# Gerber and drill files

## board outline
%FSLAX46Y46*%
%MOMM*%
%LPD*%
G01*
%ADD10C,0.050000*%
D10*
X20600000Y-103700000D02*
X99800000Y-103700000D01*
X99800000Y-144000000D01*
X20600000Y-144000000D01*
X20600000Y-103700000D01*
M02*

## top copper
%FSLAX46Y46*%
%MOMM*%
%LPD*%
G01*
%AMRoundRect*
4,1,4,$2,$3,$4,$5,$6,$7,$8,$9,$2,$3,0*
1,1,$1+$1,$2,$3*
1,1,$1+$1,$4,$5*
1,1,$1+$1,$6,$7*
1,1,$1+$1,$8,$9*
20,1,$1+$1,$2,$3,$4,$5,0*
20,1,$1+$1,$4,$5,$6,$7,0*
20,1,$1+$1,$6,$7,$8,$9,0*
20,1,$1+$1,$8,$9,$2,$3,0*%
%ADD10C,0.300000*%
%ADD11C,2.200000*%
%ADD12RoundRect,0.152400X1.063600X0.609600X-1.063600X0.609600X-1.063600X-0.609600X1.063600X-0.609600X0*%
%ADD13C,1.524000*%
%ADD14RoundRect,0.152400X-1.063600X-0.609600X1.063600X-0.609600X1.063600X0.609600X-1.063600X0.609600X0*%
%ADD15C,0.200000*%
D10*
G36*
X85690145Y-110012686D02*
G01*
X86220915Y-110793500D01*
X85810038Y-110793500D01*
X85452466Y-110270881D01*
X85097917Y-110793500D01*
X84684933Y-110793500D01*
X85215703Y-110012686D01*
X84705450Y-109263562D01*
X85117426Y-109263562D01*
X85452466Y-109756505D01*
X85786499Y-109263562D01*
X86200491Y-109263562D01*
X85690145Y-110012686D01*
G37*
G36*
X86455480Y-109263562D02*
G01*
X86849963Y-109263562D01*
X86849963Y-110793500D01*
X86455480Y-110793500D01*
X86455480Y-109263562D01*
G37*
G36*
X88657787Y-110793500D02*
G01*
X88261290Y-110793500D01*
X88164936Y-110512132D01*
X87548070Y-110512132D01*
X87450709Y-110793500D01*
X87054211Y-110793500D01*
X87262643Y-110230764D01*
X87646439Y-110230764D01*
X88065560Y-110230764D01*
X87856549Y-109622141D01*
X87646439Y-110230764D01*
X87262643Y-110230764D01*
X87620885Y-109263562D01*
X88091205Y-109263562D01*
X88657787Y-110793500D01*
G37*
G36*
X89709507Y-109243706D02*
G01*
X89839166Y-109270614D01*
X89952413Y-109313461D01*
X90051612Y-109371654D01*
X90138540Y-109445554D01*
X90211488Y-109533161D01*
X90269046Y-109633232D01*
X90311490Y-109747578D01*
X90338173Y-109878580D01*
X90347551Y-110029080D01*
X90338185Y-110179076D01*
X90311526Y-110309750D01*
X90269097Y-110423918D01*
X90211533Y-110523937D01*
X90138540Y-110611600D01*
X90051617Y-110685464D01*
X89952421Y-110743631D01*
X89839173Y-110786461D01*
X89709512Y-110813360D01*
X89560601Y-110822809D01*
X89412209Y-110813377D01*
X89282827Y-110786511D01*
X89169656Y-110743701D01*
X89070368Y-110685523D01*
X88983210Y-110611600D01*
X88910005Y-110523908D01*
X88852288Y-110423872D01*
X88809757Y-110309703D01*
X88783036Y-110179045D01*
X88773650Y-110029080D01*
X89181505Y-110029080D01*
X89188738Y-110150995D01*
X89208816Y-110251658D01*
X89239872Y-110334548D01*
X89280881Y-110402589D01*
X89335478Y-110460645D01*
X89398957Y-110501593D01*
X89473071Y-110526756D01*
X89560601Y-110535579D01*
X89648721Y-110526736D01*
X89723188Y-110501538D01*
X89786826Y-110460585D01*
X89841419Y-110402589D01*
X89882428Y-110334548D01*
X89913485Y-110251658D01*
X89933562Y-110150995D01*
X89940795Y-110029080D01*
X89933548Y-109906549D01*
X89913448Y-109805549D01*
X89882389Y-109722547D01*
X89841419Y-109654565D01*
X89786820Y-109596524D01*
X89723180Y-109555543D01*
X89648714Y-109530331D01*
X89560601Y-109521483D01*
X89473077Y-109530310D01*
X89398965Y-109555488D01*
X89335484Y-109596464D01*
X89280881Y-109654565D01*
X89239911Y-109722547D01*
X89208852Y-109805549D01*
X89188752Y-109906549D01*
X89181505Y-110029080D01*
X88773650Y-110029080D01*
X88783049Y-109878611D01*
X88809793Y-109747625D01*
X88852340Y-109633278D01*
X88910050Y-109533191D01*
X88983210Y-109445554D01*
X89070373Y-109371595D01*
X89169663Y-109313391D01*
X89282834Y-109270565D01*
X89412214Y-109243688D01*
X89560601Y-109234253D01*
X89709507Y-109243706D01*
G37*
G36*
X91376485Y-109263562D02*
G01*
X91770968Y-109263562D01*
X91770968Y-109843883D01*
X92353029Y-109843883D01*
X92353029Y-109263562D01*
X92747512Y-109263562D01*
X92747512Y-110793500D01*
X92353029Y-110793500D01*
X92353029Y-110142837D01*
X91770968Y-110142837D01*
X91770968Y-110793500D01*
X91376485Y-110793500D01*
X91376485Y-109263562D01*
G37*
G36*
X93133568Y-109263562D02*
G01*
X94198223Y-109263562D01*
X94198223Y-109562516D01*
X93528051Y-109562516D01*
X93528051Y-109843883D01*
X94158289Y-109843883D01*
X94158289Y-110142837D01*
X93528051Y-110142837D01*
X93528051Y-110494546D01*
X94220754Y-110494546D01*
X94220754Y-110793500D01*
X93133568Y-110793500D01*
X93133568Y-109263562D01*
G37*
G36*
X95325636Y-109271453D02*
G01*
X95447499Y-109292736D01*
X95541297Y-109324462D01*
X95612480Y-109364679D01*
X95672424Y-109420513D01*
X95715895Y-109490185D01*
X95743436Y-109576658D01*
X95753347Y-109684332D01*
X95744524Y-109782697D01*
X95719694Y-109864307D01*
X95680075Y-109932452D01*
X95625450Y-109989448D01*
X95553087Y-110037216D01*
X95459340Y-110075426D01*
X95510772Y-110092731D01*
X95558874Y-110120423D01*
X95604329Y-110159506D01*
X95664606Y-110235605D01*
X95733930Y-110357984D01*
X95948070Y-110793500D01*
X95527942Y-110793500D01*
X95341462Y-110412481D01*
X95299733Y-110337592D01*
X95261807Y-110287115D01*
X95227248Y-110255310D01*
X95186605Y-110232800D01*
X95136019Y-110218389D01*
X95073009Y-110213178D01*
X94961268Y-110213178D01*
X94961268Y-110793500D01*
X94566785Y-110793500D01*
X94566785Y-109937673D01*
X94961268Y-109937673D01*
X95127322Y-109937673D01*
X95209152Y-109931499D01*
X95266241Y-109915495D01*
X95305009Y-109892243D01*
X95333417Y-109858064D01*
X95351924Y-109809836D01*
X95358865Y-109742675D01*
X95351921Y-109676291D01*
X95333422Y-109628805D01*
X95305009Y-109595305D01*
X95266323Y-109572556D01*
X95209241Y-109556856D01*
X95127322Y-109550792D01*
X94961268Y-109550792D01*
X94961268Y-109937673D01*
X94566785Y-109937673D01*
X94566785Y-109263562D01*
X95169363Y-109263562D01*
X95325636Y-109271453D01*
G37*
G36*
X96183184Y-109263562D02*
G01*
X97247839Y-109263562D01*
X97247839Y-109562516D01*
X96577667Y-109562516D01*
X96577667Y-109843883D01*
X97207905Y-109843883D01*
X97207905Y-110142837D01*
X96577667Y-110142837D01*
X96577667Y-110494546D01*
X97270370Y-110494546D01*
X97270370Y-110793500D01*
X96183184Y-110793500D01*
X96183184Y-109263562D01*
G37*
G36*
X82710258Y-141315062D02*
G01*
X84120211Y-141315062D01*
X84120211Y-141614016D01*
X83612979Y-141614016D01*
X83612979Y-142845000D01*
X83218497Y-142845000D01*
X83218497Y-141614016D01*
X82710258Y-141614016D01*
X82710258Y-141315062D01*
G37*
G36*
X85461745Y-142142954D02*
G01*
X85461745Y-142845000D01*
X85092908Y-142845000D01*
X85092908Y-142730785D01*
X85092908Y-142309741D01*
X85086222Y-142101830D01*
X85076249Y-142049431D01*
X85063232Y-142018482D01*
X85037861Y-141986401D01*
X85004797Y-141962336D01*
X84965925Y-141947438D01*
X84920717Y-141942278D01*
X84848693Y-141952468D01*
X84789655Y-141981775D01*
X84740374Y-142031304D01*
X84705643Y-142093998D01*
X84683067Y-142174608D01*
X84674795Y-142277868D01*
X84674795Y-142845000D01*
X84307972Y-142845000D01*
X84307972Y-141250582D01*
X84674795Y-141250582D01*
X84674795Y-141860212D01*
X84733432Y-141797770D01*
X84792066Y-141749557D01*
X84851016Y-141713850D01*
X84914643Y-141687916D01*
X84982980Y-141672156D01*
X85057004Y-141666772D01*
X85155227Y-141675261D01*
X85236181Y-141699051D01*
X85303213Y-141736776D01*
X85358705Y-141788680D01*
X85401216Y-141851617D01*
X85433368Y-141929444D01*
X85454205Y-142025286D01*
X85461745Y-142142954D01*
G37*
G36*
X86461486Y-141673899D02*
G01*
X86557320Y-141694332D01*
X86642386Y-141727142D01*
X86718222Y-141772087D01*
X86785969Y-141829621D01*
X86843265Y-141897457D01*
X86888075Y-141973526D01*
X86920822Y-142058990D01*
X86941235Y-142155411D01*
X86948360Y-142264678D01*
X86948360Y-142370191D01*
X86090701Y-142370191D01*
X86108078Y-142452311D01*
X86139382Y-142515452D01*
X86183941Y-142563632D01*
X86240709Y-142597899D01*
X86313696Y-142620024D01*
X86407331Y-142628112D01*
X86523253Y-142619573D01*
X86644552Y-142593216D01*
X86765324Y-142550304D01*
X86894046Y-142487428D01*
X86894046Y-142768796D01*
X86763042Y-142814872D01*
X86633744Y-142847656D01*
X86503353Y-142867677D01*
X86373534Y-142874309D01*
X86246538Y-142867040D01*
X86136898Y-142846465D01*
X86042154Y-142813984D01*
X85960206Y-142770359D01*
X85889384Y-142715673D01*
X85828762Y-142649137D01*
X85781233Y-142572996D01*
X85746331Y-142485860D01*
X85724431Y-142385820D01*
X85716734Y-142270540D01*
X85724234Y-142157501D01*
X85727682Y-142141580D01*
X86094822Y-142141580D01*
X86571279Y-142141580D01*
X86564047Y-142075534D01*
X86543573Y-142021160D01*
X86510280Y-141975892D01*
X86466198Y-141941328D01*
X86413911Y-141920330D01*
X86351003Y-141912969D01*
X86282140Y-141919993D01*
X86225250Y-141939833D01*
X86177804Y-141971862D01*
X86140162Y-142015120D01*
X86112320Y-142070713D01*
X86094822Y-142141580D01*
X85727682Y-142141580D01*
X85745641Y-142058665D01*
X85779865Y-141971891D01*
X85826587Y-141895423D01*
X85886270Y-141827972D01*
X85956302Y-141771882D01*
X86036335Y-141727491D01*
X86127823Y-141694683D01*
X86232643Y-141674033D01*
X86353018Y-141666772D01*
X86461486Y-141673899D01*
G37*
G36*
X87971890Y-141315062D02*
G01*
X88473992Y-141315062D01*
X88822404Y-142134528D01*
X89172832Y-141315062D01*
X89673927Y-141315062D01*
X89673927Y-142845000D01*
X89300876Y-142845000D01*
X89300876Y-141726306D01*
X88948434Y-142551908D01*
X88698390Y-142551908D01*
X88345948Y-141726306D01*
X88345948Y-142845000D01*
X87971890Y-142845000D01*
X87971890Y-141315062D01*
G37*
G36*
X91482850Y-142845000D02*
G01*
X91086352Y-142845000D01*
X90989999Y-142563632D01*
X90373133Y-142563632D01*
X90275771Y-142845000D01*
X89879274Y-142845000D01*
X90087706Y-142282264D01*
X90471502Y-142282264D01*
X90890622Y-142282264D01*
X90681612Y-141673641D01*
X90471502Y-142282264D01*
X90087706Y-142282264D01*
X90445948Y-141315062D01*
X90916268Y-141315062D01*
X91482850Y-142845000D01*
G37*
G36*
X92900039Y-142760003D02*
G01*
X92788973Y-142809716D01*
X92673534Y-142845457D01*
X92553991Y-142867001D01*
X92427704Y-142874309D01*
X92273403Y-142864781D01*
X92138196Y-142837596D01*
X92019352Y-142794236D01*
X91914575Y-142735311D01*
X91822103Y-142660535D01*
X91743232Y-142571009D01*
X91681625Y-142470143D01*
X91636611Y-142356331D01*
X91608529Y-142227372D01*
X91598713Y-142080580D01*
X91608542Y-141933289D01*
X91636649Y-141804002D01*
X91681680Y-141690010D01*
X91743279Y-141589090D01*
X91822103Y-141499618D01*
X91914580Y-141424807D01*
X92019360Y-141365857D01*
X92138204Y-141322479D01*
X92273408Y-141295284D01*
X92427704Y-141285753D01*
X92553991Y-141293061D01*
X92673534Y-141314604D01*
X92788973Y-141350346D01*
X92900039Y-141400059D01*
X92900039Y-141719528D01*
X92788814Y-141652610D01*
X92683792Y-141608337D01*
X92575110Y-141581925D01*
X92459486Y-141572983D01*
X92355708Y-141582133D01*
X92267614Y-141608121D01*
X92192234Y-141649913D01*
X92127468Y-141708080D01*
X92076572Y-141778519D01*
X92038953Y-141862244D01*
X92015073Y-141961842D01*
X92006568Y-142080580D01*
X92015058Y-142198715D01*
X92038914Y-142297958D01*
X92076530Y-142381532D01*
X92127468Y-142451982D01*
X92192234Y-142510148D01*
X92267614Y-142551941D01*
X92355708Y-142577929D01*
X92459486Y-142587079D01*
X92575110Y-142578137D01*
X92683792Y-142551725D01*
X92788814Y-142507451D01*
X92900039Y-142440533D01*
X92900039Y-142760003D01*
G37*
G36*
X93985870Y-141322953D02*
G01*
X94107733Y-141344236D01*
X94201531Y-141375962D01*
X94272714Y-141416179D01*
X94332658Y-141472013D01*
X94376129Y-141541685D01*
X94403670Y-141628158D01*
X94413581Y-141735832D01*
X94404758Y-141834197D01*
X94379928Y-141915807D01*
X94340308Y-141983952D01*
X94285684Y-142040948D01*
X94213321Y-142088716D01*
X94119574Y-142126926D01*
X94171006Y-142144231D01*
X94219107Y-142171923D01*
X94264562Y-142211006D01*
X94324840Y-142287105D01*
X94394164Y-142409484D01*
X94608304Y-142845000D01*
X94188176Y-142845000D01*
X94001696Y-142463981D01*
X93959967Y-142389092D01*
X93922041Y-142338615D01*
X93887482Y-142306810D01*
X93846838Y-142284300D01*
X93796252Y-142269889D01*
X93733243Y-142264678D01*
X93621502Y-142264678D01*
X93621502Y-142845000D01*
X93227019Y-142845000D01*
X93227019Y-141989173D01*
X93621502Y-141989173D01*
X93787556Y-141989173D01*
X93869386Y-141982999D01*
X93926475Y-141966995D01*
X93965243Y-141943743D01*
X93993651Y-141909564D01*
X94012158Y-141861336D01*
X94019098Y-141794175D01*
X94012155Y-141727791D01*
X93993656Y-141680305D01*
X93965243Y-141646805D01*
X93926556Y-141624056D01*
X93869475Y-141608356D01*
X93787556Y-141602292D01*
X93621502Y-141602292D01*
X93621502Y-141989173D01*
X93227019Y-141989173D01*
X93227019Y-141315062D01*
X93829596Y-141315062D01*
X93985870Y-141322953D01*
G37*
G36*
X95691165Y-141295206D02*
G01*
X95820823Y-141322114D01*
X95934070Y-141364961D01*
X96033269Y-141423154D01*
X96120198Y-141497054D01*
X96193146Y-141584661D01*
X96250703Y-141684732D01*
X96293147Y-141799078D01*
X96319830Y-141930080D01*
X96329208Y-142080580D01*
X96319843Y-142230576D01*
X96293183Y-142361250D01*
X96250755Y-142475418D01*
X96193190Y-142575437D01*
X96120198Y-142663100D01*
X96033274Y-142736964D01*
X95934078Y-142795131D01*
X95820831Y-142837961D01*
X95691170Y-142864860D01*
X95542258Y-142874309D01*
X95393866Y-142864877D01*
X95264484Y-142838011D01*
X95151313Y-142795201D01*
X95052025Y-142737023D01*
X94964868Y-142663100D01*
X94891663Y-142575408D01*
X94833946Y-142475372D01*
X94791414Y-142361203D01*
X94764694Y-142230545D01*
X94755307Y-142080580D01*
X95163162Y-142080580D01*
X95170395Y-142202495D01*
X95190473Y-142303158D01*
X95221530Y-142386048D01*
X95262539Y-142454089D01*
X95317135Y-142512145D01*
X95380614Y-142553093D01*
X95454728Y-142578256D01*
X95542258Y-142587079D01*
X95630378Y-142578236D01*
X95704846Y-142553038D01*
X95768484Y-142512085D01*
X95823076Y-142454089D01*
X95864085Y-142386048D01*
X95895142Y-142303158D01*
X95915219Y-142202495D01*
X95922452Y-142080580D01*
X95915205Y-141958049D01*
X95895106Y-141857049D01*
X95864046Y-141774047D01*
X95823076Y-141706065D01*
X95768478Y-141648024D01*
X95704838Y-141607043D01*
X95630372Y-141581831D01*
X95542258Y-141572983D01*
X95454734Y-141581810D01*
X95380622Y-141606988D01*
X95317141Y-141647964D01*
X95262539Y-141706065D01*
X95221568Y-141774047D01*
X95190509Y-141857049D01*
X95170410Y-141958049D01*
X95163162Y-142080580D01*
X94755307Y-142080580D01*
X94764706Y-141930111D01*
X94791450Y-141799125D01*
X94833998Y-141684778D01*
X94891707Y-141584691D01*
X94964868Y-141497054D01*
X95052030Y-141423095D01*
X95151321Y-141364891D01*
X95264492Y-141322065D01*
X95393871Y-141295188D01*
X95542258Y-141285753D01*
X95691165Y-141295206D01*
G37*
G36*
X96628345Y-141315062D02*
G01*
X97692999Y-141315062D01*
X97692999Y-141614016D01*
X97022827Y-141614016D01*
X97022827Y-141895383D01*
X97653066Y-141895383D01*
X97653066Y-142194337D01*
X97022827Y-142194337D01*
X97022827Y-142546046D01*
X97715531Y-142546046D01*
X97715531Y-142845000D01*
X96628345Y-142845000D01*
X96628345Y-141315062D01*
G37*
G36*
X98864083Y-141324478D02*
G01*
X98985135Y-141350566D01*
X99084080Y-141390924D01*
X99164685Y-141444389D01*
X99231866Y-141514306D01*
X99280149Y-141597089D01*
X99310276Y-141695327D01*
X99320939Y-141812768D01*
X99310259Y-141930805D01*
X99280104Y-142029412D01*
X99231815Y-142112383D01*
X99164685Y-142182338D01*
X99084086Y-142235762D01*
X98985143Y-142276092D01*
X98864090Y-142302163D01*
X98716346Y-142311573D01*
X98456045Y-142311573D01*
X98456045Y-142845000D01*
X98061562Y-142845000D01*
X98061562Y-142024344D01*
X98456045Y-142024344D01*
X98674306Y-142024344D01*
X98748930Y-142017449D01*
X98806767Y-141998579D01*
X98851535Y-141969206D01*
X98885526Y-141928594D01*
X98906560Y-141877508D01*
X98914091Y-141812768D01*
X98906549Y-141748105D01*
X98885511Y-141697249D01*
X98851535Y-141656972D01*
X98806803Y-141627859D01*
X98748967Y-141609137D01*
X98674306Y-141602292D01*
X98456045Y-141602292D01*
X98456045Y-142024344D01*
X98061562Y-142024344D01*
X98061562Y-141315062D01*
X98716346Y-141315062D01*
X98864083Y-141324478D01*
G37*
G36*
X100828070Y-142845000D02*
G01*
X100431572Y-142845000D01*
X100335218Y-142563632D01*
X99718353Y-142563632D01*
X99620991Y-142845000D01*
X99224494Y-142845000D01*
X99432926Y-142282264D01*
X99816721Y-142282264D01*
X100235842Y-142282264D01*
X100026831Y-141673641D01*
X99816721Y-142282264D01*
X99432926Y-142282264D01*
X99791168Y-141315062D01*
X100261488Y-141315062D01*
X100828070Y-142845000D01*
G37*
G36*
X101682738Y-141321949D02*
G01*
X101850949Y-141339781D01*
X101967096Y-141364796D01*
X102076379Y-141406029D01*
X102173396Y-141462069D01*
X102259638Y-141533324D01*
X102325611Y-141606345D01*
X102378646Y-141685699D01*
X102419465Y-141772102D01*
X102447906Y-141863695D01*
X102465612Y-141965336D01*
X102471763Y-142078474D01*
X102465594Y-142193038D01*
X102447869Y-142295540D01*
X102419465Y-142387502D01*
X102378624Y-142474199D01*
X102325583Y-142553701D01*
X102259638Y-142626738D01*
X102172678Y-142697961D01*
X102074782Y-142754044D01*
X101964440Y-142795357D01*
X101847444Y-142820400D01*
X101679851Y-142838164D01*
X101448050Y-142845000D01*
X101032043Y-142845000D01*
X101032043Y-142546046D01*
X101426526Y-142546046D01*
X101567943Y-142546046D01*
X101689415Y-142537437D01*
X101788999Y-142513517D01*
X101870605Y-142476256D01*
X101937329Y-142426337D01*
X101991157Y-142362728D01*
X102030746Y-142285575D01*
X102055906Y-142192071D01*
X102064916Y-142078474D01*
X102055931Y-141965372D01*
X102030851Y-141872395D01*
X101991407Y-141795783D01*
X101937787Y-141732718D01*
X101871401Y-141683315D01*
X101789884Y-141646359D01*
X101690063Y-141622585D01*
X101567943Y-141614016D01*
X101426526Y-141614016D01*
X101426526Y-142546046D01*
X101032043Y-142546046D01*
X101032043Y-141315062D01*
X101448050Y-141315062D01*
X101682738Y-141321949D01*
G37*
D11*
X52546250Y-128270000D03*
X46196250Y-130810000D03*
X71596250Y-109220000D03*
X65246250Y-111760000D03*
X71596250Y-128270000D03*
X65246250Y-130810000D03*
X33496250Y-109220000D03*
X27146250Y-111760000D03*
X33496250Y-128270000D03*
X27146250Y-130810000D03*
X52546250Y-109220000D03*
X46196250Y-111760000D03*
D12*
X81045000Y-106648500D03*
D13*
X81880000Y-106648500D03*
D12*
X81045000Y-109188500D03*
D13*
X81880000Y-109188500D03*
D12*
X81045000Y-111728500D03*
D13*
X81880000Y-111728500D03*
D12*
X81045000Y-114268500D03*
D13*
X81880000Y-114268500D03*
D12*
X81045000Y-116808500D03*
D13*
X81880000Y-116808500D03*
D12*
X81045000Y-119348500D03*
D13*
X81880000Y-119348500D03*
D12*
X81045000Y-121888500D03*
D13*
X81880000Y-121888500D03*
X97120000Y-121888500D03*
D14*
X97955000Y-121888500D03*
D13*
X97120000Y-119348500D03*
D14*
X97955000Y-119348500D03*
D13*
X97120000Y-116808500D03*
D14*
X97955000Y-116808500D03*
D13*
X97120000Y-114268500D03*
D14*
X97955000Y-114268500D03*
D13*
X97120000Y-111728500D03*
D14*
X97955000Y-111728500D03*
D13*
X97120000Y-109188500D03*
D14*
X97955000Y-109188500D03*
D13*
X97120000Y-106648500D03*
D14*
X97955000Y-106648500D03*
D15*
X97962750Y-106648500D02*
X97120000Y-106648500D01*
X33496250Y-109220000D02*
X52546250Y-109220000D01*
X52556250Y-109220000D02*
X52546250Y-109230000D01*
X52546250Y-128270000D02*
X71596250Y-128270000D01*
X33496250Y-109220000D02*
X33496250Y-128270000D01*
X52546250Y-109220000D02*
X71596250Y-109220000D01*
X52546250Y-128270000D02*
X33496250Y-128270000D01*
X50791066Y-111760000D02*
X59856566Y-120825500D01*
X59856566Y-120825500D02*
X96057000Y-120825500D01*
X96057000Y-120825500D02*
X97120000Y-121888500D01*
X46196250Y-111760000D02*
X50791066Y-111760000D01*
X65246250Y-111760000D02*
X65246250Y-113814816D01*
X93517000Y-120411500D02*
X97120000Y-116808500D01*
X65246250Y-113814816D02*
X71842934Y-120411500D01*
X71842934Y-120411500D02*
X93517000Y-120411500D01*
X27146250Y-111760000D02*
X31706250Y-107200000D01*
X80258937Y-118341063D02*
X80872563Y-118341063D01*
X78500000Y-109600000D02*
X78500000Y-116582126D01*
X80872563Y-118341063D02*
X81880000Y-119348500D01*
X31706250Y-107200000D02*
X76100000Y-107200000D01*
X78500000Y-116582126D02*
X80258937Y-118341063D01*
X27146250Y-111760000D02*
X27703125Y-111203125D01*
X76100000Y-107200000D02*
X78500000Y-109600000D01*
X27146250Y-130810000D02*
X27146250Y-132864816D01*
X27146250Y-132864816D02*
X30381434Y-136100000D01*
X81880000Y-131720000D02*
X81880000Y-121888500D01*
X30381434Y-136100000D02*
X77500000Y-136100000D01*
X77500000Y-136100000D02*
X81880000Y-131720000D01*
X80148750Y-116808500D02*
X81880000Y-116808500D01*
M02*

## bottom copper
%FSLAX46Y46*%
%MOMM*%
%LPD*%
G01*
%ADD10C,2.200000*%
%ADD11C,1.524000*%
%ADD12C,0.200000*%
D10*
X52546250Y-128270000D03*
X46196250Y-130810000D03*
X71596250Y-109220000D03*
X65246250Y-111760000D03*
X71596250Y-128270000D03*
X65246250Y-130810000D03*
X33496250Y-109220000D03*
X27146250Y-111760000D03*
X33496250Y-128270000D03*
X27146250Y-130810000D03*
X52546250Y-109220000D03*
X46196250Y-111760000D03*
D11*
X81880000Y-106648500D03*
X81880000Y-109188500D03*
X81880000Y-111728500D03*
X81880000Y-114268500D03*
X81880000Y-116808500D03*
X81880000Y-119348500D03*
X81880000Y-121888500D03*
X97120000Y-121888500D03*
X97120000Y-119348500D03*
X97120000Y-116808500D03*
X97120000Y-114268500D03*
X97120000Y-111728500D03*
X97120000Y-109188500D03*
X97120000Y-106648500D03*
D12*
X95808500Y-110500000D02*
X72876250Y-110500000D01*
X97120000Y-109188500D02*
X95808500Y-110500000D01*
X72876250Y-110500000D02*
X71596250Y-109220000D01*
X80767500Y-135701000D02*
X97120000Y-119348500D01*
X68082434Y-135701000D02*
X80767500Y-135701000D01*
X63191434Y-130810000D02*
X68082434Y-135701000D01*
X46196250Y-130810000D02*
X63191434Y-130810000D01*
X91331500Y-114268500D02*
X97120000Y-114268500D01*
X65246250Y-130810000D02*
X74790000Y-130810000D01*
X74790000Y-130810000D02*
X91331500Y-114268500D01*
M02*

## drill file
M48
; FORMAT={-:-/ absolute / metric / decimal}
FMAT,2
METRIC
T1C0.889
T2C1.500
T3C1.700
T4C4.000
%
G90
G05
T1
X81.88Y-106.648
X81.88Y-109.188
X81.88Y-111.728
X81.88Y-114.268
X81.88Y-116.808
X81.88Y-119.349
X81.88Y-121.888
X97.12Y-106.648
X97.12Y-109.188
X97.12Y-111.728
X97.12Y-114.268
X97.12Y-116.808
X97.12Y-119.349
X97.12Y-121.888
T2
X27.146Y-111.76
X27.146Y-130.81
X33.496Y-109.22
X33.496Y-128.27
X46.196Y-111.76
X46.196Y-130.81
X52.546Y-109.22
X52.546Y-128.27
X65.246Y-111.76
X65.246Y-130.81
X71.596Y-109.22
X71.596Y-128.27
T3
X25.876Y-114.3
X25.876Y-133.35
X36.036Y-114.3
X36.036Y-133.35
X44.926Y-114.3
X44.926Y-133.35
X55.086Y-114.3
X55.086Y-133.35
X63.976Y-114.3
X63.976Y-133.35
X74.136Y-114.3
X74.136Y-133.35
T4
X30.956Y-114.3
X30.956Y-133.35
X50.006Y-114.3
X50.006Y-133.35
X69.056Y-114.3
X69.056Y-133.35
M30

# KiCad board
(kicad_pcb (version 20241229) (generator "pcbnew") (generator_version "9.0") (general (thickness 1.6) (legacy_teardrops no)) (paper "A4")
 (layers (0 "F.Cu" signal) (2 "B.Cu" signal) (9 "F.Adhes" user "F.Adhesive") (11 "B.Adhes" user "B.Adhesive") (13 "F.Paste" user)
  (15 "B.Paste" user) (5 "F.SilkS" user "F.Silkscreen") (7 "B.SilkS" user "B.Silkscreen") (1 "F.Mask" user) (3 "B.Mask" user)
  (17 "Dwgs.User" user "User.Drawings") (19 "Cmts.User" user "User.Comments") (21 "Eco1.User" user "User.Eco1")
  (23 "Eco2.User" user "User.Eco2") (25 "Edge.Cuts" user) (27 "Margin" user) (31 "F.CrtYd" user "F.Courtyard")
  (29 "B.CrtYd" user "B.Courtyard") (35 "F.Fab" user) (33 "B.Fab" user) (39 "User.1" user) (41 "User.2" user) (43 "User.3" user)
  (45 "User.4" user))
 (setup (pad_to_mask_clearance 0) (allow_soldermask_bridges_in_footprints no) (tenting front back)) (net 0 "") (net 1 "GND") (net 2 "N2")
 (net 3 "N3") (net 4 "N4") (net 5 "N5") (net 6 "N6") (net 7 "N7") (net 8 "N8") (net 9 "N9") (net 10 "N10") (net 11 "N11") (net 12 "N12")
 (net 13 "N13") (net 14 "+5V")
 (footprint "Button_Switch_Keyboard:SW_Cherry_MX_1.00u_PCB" (layer "F.Cu") (at 52.54625 128.27)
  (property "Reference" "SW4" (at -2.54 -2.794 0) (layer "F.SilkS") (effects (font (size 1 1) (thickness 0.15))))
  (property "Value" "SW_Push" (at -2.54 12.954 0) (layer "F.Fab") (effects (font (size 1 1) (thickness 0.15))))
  (pad "" np_thru_hole circle (at -7.62 5.08) (size 1.7 1.7) (drill 1.7) (layers "*.Cu" "*.Mask"))
  (pad "" np_thru_hole circle (at -2.54 5.08) (size 4 4) (drill 4) (layers "*.Cu" "*.Mask"))
  (pad "" np_thru_hole circle (at 2.54 5.08) (size 1.7 1.7) (drill 1.7) (layers "*.Cu" "*.Mask"))
  (pad "1" thru_hole circle (at 0 0) (size 2.2 2.2) (drill 1.5) (layers "*.Cu" "*.Mask") (remove_unused_layers no) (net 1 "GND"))
  (pad "2" thru_hole circle (at -6.35 2.54) (size 2.2 2.2) (drill 1.5) (layers "*.Cu" "*.Mask") (remove_unused_layers no) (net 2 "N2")))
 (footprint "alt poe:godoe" (layer "F.Cu") (at 90.7 131.5)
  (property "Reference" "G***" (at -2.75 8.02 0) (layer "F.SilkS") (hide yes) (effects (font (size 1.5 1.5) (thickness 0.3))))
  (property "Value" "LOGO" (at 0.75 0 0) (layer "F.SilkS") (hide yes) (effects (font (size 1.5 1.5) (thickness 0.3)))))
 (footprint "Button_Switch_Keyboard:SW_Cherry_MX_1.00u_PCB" (layer "F.Cu") (at 71.59625 109.22)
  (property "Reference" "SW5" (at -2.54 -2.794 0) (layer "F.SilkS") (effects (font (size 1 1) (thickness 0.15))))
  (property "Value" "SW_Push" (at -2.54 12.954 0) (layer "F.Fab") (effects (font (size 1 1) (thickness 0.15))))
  (pad "" np_thru_hole circle (at -7.62 5.08) (size 1.7 1.7) (drill 1.7) (layers "*.Cu" "*.Mask"))
  (pad "" np_thru_hole circle (at -2.54 5.08) (size 4 4) (drill 4) (layers "*.Cu" "*.Mask"))
  (pad "" np_thru_hole circle (at 2.54 5.08) (size 1.7 1.7) (drill 1.7) (layers "*.Cu" "*.Mask"))
  (pad "1" thru_hole circle (at 0 0) (size 2.2 2.2) (drill 1.5) (layers "*.Cu" "*.Mask") (remove_unused_layers no) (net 1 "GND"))
  (pad "2" thru_hole circle (at -6.35 2.54) (size 2.2 2.2) (drill 1.5) (layers "*.Cu" "*.Mask") (remove_unused_layers no) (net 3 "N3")))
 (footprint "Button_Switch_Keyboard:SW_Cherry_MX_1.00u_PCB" (layer "F.Cu") (at 71.59625 128.27)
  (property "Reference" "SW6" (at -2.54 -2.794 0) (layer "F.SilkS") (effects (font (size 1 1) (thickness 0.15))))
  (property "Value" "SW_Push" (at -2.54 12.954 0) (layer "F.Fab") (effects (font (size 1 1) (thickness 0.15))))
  (pad "" np_thru_hole circle (at -7.62 5.08) (size 1.7 1.7) (drill 1.7) (layers "*.Cu" "*.Mask"))
  (pad "" np_thru_hole circle (at -2.54 5.08) (size 4 4) (drill 4) (layers "*.Cu" "*.Mask"))
  (pad "" np_thru_hole circle (at 2.54 5.08) (size 1.7 1.7) (drill 1.7) (layers "*.Cu" "*.Mask"))
  (pad "1" thru_hole circle (at 0 0) (size 2.2 2.2) (drill 1.5) (layers "*.Cu" "*.Mask") (remove_unused_layers no) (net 1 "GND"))
  (pad "2" thru_hole circle (at -6.35 2.54) (size 2.2 2.2) (drill 1.5) (layers "*.Cu" "*.Mask") (remove_unused_layers no) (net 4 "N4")))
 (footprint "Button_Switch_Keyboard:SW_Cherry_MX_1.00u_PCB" (layer "F.Cu") (at 33.49625 109.22)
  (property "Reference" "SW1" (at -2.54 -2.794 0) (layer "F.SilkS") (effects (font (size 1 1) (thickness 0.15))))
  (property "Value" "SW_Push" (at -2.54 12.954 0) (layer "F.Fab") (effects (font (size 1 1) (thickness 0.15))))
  (pad "" np_thru_hole circle (at -7.62 5.08) (size 1.7 1.7) (drill 1.7) (layers "*.Cu" "*.Mask"))
  (pad "" np_thru_hole circle (at -2.54 5.08) (size 4 4) (drill 4) (layers "*.Cu" "*.Mask"))
  (pad "" np_thru_hole circle (at 2.54 5.08) (size 1.7 1.7) (drill 1.7) (layers "*.Cu" "*.Mask"))
  (pad "1" thru_hole circle (at 0 0) (size 2.2 2.2) (drill 1.5) (layers "*.Cu" "*.Mask") (remove_unused_layers no) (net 1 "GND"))
  (pad "2" thru_hole circle (at -6.35 2.54) (size 2.2 2.2) (drill 1.5) (layers "*.Cu" "*.Mask") (remove_unused_layers no) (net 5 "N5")))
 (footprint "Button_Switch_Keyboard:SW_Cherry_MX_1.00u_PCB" (layer "F.Cu") (at 33.49625 128.27)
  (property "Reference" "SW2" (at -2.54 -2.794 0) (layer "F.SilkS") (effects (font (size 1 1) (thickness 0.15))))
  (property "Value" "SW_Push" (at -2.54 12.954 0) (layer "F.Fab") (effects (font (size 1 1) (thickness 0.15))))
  (pad "" np_thru_hole circle (at -7.62 5.08) (size 1.7 1.7) (drill 1.7) (layers "*.Cu" "*.Mask"))
  (pad "" np_thru_hole circle (at -2.54 5.08) (size 4 4) (drill 4) (layers "*.Cu" "*.Mask"))
  (pad "" np_thru_hole circle (at 2.54 5.08) (size 1.7 1.7) (drill 1.7) (layers "*.Cu" "*.Mask"))
  (pad "1" thru_hole circle (at 0 0) (size 2.2 2.2) (drill 1.5) (layers "*.Cu" "*.Mask") (remove_unused_layers no) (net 1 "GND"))
  (pad "2" thru_hole circle (at -6.35 2.54) (size 2.2 2.2) (drill 1.5) (layers "*.Cu" "*.Mask") (remove_unused_layers no) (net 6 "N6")))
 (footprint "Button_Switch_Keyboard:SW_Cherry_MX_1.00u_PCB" (layer "F.Cu") (at 52.54625 109.22)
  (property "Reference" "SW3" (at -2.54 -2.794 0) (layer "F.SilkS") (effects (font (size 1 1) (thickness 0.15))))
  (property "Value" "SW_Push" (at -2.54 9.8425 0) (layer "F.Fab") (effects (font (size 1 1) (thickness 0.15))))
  (pad "" np_thru_hole circle (at -7.62 5.08) (size 1.7 1.7) (drill 1.7) (layers "*.Cu" "*.Mask"))
  (pad "" np_thru_hole circle (at -2.54 5.08) (size 4 4) (drill 4) (layers "*.Cu" "*.Mask"))
  (pad "" np_thru_hole circle (at 2.54 5.08) (size 1.7 1.7) (drill 1.7) (layers "*.Cu" "*.Mask"))
  (pad "1" thru_hole circle (at 0 0) (size 2.2 2.2) (drill 1.5) (layers "*.Cu" "*.Mask") (remove_unused_layers no) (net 1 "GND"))
  (pad "2" thru_hole circle (at -6.35 2.54) (size 2.2 2.2) (drill 1.5) (layers "*.Cu" "*.Mask") (remove_unused_layers no) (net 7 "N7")))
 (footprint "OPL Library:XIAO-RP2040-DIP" (layer "F.Cu") (at 89.5 114.2685)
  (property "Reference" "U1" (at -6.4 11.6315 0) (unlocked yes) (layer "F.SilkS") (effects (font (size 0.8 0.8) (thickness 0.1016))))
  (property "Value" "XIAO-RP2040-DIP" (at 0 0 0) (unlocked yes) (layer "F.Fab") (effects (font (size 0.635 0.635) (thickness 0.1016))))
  (pad "1" smd roundrect (at -8.455 -7.62 180) (size 2.432 1.524) (layers "F.Cu" "F.Mask") (roundrect_rratio 0.1) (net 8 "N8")
   (thermal_bridge_angle 45))
  (pad "1" thru_hole circle (at -7.62 -7.62 180) (size 1.524 1.524) (drill 0.889) (layers "*.Cu" "*.Mask") (remove_unused_layers no)
   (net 8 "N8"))
  (pad "2" smd roundrect (at -8.455 -5.08 180) (size 2.432 1.524) (layers "F.Cu" "F.Mask") (roundrect_rratio 0.1) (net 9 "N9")
   (thermal_bridge_angle 45))
  (pad "2" thru_hole circle (at -7.62 -5.08 180) (size 1.524 1.524) (drill 0.889) (layers "*.Cu" "*.Mask") (remove_unused_layers no)
   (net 9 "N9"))
  (pad "3" smd roundrect (at -8.455 -2.54 180) (size 2.432 1.524) (layers "F.Cu" "F.Mask") (roundrect_rratio 0.1) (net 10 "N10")
   (thermal_bridge_angle 45))
  (pad "3" thru_hole circle (at -7.62 -2.54 180) (size 1.524 1.524) (drill 0.889) (layers "*.Cu" "*.Mask") (remove_unused_layers no)
   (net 10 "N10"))
  (pad "4" smd roundrect (at -8.455 0 180) (size 2.432 1.524) (layers "F.Cu" "F.Mask") (roundrect_rratio 0.1) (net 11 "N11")
   (thermal_bridge_angle 45))
  (pad "4" thru_hole circle (at -7.62 0 180) (size 1.524 1.524) (drill 0.889) (layers "*.Cu" "*.Mask") (remove_unused_layers no)
   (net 11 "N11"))
  (pad "5" smd roundrect (at -8.455 2.54 180) (size 2.432 1.524) (layers "F.Cu" "F.Mask") (roundrect_rratio 0.1) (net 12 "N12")
   (thermal_bridge_angle 45))
  (pad "5" thru_hole circle (at -7.62 2.54 180) (size 1.524 1.524) (drill 0.889) (layers "*.Cu" "*.Mask") (remove_unused_layers no)
   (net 12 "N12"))
  (pad "6" smd roundrect (at -8.455 5.08 180) (size 2.432 1.524) (layers "F.Cu" "F.Mask") (roundrect_rratio 0.1) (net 5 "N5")
   (thermal_bridge_angle 45))
  (pad "6" thru_hole circle (at -7.62 5.08 180) (size 1.524 1.524) (drill 0.889) (layers "*.Cu" "*.Mask") (remove_unused_layers no)
   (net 5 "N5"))
  (pad "7" smd roundrect (at -8.455 7.62 180) (size 2.432 1.524) (layers "F.Cu" "F.Mask") (roundrect_rratio 0.1) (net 6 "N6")
   (thermal_bridge_angle 45))
  (pad "7" thru_hole circle (at -7.62 7.62 180) (size 1.524 1.524) (drill 0.889) (layers "*.Cu" "*.Mask") (remove_unused_layers no)
   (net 6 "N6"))
  (pad "8" thru_hole circle (at 7.62 7.62) (size 1.524 1.524) (drill 0.889) (layers "*.Cu" "*.Mask") (remove_unused_layers no) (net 7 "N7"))
  (pad "8" smd roundrect (at 8.455 7.62) (size 2.432 1.524) (layers "F.Cu" "F.Mask") (roundrect_rratio 0.1) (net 7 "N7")
   (thermal_bridge_angle 45))
  (pad "9" thru_hole circle (at 7.62 5.08) (size 1.524 1.524) (drill 0.889) (layers "*.Cu" "*.Mask") (remove_unused_layers no) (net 2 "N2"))
  (pad "9" smd roundrect (at 8.455 5.08) (size 2.432 1.524) (layers "F.Cu" "F.Mask") (roundrect_rratio 0.1) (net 2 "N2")
   (thermal_bridge_angle 45))
  (pad "10" thru_hole circle (at 7.62 2.54) (size 1.524 1.524) (drill 0.889) (layers "*.Cu" "*.Mask") (remove_unused_layers no) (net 3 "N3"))
  (pad "10" smd roundrect (at 8.455 2.54) (size 2.432 1.524) (layers "F.Cu" "F.Mask") (roundrect_rratio 0.1) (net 3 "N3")
   (thermal_bridge_angle 45))
  (pad "11" thru_hole circle (at 7.62 0) (size 1.524 1.524) (drill 0.889) (layers "*.Cu" "*.Mask") (remove_unused_layers no) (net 4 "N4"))
  (pad "11" smd roundrect (at 8.455 0) (size 2.432 1.524) (layers "F.Cu" "F.Mask") (roundrect_rratio 0.1) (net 4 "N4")
   (thermal_bridge_angle 45))
  (pad "12" thru_hole circle (at 7.62 -2.54) (size 1.524 1.524) (drill 0.889) (layers "*.Cu" "*.Mask") (remove_unused_layers no)
   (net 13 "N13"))
  (pad "12" smd roundrect (at 8.455 -2.54) (size 2.432 1.524) (layers "F.Cu" "F.Mask") (roundrect_rratio 0.1) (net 13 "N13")
   (thermal_bridge_angle 45))
  (pad "13" thru_hole circle (at 7.62 -5.08) (size 1.524 1.524) (drill 0.889) (layers "*.Cu" "*.Mask") (remove_unused_layers no)
   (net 1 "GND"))
  (pad "13" smd roundrect (at 8.455 -5.08) (size 2.432 1.524) (layers "F.Cu" "F.Mask") (roundrect_rratio 0.1) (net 1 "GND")
   (thermal_bridge_angle 45))
  (pad "14" thru_hole circle (at 7.62 -7.62) (size 1.524 1.524) (drill 0.889) (layers "*.Cu" "*.Mask") (remove_unused_layers no)
   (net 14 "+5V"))
  (pad "14" smd roundrect (at 8.455 -7.62) (size 2.432 1.524) (layers "F.Cu" "F.Mask") (roundrect_rratio 0.1) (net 14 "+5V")
   (thermal_bridge_angle 45)))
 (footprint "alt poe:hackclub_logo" (layer "F.Cu") (at 85.3 139.1)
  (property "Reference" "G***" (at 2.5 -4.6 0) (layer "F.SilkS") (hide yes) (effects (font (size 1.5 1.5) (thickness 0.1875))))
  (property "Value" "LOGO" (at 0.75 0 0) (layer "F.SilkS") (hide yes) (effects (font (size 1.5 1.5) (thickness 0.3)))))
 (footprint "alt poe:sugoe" (layer "B.Cu") (at 87.4 131.6 180)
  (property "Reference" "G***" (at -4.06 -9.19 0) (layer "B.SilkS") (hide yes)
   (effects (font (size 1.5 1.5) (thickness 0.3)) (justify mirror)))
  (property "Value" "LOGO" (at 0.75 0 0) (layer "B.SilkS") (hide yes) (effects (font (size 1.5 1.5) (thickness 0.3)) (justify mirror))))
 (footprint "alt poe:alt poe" (layer "B.Cu") (at 43.4 121.9 180)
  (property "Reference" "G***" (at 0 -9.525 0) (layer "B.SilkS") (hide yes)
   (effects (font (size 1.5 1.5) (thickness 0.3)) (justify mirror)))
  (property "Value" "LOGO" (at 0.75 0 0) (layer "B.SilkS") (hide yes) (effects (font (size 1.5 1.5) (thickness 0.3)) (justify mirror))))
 (gr_rect (start 20.6 103.7) (end 99.8 144) (stroke (width 0.05) (type default)) (fill no) (layer "Edge.Cuts"))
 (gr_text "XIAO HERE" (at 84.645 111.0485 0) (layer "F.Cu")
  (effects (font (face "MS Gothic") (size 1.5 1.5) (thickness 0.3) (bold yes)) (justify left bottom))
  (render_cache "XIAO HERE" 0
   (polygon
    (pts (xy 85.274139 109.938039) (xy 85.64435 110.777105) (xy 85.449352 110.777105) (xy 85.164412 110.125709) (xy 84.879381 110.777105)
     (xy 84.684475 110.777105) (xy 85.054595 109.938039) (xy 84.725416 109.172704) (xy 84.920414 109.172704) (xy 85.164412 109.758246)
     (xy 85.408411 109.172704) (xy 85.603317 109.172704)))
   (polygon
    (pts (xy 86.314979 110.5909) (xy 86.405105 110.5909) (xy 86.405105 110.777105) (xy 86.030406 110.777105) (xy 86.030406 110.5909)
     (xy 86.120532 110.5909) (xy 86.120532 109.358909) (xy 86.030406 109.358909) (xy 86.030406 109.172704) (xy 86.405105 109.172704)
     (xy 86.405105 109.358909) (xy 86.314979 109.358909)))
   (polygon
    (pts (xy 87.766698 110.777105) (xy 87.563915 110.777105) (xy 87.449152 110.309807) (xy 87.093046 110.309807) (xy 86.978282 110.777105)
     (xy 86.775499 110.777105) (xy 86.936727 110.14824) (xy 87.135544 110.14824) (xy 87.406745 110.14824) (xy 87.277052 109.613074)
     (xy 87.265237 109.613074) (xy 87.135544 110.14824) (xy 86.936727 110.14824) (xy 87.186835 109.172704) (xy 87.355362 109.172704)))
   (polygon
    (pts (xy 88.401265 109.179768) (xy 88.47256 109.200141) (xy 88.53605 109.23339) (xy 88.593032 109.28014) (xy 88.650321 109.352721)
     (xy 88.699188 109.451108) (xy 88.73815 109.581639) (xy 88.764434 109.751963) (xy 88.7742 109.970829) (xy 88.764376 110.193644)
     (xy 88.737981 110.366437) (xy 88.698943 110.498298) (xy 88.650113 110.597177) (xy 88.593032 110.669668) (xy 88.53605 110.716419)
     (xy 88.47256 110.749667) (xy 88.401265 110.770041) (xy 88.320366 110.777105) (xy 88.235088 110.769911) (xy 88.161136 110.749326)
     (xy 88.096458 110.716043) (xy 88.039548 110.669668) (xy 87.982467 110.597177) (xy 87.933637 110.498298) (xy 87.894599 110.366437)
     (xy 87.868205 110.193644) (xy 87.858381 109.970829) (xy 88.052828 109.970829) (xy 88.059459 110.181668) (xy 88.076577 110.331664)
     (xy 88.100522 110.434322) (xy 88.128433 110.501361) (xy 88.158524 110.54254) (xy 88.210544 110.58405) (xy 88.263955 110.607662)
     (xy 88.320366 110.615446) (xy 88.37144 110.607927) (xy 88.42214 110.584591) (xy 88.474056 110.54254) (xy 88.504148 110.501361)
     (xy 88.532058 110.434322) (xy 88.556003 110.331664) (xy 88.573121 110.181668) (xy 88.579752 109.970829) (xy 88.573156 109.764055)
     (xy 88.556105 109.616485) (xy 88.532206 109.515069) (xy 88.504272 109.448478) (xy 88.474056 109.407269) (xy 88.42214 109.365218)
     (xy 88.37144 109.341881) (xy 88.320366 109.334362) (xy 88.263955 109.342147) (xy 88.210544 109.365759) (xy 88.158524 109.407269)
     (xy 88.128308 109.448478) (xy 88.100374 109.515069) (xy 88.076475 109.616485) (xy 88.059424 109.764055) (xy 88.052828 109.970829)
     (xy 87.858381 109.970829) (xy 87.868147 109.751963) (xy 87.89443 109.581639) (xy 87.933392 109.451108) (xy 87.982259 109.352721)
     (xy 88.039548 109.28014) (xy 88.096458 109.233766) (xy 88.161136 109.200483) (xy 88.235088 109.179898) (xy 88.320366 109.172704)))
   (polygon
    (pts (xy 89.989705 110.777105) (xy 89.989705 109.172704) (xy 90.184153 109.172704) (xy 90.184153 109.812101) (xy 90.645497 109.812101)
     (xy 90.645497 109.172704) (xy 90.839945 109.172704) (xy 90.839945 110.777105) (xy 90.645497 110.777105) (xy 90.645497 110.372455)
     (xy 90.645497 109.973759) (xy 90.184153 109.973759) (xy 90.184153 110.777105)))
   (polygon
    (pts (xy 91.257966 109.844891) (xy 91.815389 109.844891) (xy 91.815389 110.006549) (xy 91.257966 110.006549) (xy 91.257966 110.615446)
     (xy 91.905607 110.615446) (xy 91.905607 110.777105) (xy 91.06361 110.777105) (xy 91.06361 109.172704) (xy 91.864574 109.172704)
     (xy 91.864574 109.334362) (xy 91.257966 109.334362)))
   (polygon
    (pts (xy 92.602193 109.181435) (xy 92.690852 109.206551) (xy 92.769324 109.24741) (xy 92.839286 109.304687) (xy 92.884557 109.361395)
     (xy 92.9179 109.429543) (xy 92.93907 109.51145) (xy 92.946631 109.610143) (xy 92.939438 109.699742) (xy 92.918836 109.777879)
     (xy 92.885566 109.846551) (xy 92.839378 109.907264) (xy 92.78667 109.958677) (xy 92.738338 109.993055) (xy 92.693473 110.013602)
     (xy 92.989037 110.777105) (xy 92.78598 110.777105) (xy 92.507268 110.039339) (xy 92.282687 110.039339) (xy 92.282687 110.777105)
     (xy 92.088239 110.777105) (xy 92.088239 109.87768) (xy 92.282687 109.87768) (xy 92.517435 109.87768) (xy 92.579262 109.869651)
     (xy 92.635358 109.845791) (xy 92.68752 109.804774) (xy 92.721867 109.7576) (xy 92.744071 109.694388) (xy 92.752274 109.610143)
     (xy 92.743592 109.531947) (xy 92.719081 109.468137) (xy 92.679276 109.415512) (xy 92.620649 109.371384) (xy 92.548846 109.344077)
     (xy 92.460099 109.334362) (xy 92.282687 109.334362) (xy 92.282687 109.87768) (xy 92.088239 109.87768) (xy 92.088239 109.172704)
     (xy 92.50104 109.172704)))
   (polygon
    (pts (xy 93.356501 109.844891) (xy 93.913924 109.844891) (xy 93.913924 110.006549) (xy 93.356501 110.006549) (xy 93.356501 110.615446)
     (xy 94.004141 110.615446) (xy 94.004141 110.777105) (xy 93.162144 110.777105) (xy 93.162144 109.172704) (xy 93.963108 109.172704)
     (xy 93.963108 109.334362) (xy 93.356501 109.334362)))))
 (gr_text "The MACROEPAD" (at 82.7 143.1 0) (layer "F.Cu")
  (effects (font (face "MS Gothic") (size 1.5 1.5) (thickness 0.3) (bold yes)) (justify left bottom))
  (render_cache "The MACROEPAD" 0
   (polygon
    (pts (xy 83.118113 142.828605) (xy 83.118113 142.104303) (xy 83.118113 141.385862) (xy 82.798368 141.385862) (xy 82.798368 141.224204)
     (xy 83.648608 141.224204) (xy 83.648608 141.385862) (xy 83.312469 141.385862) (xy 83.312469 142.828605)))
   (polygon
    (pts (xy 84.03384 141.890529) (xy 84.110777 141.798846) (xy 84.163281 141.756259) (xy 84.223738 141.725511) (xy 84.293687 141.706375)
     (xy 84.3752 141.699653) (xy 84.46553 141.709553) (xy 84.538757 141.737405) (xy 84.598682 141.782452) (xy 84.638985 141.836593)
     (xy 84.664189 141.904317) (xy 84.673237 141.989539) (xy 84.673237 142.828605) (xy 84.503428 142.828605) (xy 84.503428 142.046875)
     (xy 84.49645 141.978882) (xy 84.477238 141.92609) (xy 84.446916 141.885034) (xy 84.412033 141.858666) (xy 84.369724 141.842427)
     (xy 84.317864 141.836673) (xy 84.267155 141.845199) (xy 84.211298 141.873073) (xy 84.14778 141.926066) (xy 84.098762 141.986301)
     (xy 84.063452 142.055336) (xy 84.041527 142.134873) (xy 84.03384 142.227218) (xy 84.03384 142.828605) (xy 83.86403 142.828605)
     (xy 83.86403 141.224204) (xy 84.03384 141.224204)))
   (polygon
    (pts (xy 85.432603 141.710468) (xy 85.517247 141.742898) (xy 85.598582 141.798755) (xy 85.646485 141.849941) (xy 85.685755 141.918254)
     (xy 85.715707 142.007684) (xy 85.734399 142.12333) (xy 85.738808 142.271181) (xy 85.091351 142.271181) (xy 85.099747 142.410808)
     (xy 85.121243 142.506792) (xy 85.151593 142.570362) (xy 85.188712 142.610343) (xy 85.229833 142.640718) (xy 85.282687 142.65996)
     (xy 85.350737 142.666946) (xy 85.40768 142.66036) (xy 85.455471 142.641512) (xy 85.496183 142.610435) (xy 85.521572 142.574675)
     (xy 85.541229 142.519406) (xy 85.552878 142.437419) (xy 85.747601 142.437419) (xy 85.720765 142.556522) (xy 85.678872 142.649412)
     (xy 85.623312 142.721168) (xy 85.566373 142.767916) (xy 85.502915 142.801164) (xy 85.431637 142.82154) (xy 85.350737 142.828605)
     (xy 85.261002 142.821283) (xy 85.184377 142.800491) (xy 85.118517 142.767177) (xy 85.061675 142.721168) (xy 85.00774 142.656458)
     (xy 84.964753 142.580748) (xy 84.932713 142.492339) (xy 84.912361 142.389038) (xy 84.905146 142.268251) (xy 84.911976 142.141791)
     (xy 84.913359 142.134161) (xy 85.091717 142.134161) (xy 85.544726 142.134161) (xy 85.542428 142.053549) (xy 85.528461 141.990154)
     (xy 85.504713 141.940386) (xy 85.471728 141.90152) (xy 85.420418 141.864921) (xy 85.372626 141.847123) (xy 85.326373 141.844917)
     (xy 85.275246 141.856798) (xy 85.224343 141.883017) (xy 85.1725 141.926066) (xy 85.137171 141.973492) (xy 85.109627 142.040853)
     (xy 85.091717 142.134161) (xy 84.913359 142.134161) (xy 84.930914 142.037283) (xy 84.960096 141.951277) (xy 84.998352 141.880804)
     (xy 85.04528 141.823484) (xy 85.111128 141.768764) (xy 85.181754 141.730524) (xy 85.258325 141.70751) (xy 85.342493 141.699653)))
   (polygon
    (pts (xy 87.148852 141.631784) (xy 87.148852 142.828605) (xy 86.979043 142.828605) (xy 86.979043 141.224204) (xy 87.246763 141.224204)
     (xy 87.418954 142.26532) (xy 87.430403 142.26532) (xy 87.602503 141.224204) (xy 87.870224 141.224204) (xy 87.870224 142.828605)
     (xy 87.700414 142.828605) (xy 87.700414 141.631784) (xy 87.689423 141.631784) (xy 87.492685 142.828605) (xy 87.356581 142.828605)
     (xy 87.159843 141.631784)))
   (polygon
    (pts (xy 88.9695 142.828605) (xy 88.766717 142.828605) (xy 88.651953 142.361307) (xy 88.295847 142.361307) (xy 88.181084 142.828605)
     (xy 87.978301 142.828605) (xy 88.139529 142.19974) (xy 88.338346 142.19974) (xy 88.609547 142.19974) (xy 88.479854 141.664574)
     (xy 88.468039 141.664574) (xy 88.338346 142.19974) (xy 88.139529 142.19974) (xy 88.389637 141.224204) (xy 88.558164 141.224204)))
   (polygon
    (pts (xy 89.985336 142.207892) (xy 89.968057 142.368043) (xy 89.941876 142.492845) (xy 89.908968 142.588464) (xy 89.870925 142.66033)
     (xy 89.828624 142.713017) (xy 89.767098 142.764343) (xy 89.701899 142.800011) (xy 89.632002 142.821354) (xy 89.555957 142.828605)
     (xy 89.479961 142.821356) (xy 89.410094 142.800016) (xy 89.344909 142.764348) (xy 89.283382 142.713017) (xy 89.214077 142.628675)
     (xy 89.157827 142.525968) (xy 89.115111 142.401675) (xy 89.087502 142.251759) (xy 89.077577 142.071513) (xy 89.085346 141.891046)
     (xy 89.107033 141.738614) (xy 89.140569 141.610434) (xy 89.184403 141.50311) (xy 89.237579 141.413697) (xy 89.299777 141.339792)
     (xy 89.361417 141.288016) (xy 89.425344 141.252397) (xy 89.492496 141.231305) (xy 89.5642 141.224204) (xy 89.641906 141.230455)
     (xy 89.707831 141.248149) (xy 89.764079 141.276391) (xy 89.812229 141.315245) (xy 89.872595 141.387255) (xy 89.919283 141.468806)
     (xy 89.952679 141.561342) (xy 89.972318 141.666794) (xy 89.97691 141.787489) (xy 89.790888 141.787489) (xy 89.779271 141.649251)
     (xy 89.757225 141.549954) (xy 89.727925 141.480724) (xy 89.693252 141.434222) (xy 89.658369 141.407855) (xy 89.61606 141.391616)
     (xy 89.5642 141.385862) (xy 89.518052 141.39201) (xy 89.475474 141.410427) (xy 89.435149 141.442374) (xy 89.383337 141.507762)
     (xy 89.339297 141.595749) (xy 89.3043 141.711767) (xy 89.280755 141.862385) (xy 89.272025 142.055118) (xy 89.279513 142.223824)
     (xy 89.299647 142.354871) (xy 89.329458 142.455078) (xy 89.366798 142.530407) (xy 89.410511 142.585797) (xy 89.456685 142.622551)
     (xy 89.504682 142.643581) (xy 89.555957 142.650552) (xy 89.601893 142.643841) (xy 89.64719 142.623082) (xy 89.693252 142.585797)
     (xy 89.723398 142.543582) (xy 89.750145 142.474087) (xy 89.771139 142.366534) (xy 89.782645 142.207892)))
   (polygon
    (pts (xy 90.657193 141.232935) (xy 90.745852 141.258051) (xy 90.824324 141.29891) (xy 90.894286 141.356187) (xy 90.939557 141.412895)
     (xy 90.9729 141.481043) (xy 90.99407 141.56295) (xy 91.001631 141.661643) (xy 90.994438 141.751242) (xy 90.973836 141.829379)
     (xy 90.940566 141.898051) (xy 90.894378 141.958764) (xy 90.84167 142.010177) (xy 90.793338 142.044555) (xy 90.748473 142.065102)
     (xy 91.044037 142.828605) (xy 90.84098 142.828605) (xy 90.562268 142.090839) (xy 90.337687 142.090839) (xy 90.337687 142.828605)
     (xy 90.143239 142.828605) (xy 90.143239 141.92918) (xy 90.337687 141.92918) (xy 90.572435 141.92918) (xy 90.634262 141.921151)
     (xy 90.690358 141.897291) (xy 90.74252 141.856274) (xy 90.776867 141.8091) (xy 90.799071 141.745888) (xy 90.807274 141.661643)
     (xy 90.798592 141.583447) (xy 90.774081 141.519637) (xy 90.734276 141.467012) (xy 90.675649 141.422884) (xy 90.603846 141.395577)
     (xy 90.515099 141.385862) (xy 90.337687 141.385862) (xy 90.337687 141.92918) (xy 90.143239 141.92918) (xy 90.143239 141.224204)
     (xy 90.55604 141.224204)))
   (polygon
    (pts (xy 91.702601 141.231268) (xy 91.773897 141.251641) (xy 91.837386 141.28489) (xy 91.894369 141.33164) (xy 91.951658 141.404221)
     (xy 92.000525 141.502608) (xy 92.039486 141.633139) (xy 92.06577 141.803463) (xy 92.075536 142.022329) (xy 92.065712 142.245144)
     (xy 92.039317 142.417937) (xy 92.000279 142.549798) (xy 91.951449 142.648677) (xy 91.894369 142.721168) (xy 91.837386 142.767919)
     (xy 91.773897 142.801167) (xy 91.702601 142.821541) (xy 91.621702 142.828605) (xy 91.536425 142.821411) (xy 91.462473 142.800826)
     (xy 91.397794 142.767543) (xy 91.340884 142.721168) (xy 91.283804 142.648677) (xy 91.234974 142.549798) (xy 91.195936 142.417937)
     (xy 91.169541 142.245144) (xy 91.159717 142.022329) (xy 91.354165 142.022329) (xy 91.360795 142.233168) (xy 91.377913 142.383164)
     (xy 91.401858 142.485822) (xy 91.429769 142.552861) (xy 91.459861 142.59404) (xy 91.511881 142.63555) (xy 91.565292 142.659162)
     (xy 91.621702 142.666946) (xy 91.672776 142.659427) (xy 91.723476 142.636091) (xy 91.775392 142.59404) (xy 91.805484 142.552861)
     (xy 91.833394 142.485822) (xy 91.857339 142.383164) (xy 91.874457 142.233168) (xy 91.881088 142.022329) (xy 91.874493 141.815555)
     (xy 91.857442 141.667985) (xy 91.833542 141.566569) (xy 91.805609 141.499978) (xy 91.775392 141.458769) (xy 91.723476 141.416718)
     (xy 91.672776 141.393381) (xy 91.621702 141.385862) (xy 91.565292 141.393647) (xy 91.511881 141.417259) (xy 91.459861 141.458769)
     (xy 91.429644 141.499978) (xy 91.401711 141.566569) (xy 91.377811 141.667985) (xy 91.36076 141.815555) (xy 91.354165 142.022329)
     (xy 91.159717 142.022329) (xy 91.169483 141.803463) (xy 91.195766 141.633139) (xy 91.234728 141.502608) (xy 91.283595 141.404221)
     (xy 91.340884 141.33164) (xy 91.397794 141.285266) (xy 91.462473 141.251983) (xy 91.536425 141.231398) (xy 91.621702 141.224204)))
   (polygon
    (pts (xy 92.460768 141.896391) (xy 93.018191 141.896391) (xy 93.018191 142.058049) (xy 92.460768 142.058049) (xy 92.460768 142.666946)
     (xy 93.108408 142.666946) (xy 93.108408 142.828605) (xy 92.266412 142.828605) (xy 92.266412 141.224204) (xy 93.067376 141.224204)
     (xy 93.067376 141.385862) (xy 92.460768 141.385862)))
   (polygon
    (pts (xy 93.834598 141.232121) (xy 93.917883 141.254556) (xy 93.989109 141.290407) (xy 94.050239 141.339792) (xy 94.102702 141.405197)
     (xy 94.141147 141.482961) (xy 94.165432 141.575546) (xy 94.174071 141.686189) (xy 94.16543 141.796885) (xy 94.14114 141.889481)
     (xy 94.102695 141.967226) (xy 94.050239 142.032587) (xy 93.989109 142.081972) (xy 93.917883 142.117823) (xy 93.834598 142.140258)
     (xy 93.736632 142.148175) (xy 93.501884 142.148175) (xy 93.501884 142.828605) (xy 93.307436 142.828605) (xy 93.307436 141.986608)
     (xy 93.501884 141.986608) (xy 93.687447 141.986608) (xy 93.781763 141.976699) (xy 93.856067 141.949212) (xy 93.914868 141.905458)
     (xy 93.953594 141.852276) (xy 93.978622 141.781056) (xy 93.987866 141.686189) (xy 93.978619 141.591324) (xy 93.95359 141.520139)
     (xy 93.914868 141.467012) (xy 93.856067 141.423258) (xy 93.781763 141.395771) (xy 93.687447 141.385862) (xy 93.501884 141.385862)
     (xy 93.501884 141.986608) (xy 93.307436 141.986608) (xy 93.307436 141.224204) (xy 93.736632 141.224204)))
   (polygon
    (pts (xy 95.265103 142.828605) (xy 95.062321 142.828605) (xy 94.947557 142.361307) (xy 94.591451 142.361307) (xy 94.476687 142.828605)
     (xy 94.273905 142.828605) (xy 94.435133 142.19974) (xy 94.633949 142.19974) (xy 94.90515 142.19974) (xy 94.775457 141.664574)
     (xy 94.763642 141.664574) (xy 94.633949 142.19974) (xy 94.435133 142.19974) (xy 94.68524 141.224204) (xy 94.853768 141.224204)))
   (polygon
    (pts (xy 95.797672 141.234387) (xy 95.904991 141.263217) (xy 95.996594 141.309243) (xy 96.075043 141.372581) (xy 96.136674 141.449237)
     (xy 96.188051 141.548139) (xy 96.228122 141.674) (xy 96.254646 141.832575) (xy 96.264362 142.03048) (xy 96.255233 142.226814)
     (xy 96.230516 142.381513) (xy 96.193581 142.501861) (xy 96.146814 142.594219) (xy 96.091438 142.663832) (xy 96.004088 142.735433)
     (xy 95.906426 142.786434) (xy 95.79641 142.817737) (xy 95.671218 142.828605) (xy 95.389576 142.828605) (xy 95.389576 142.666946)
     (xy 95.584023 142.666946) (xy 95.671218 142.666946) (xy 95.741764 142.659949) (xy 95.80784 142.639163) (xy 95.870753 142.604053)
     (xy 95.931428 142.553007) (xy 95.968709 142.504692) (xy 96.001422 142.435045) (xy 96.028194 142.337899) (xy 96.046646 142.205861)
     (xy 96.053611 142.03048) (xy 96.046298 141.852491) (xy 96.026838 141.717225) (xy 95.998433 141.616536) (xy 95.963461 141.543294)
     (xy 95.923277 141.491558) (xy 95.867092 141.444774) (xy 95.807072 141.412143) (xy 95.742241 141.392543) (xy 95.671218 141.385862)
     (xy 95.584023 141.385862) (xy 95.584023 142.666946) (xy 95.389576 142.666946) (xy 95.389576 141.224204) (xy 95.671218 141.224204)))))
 (segment (start 97.96275 106.6485) (end 97.12 106.6485) (width 0.2) (layer "F.Cu") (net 14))
 (segment (start 33.49625 109.22) (end 52.54625 109.22) (width 0.2) (layer "F.Cu") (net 1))
 (segment (start 52.55625 109.22) (end 52.54625 109.23) (width 0.2) (layer "F.Cu") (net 1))
 (segment (start 52.54625 128.27) (end 71.59625 128.27) (width 0.2) (layer "F.Cu") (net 1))
 (segment (start 33.49625 109.22) (end 33.49625 128.27) (width 0.2) (layer "F.Cu") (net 1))
 (segment (start 52.54625 109.22) (end 71.59625 109.22) (width 0.2) (layer "F.Cu") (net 1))
 (segment (start 52.54625 128.27) (end 33.49625 128.27) (width 0.2) (layer "F.Cu") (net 1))
 (segment (start 95.8085 110.5) (end 72.87625 110.5) (width 0.2) (layer "B.Cu") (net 1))
 (segment (start 97.12 109.1885) (end 95.8085 110.5) (width 0.2) (layer "B.Cu") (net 1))
 (segment (start 72.87625 110.5) (end 71.59625 109.22) (width 0.2) (layer "B.Cu") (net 1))
 (segment (start 50.791066 111.76) (end 59.856566 120.8255) (width 0.2) (layer "F.Cu") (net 7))
 (segment (start 59.856566 120.8255) (end 96.057 120.8255) (width 0.2) (layer "F.Cu") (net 7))
 (segment (start 96.057 120.8255) (end 97.12 121.8885) (width 0.2) (layer "F.Cu") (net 7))
 (segment (start 46.19625 111.76) (end 50.791066 111.76) (width 0.2) (layer "F.Cu") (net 7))
 (segment (start 80.7675 135.701) (end 97.12 119.3485) (width 0.2) (layer "B.Cu") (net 2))
 (segment (start 68.082434 135.701) (end 80.7675 135.701) (width 0.2) (layer "B.Cu") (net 2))
 (segment (start 63.191434 130.81) (end 68.082434 135.701) (width 0.2) (layer "B.Cu") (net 2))
 (segment (start 46.19625 130.81) (end 63.191434 130.81) (width 0.2) (layer "B.Cu") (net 2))
 (segment (start 65.24625 111.76) (end 65.24625 113.814816) (width 0.2) (layer "F.Cu") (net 3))
 (segment (start 93.517 120.4115) (end 97.12 116.8085) (width 0.2) (layer "F.Cu") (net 3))
 (segment (start 65.24625 113.814816) (end 71.842934 120.4115) (width 0.2) (layer "F.Cu") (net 3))
 (segment (start 71.842934 120.4115) (end 93.517 120.4115) (width 0.2) (layer "F.Cu") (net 3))
 (segment (start 27.14625 111.76) (end 31.70625 107.2) (width 0.2) (layer "F.Cu") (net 5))
 (segment (start 80.258937 118.341063) (end 80.872563 118.341063) (width 0.2) (layer "F.Cu") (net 5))
 (segment (start 78.5 109.6) (end 78.5 116.582126) (width 0.2) (layer "F.Cu") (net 5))
 (segment (start 80.872563 118.341063) (end 81.88 119.3485) (width 0.2) (layer "F.Cu") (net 5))
 (segment (start 31.70625 107.2) (end 76.1 107.2) (width 0.2) (layer "F.Cu") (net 5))
 (segment (start 78.5 116.582126) (end 80.258937 118.341063) (width 0.2) (layer "F.Cu") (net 5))
 (segment (start 27.14625 111.76) (end 27.703125 111.203125) (width 0.2) (layer "F.Cu") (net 5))
 (segment (start 76.1 107.2) (end 78.5 109.6) (width 0.2) (layer "F.Cu") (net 5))
 (segment (start 27.14625 130.81) (end 27.14625 132.864816) (width 0.2) (layer "F.Cu") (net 6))
 (segment (start 27.14625 132.864816) (end 30.381434 136.1) (width 0.2) (layer "F.Cu") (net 6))
 (segment (start 81.88 131.72) (end 81.88 121.8885) (width 0.2) (layer "F.Cu") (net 6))
 (segment (start 30.381434 136.1) (end 77.5 136.1) (width 0.2) (layer "F.Cu") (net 6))
 (segment (start 77.5 136.1) (end 81.88 131.72) (width 0.2) (layer "F.Cu") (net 6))
 (segment (start 91.3315 114.2685) (end 97.12 114.2685) (width 0.2) (layer "B.Cu") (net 4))
 (segment (start 65.24625 130.81) (end 74.79 130.81) (width 0.2) (layer "B.Cu") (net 4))
 (segment (start 74.79 130.81) (end 91.3315 114.2685) (width 0.2) (layer "B.Cu") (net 4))
 (segment (start 80.14875 116.8085) (end 81.88 116.8085) (width 0.2) (layer "F.Cu") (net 12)))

